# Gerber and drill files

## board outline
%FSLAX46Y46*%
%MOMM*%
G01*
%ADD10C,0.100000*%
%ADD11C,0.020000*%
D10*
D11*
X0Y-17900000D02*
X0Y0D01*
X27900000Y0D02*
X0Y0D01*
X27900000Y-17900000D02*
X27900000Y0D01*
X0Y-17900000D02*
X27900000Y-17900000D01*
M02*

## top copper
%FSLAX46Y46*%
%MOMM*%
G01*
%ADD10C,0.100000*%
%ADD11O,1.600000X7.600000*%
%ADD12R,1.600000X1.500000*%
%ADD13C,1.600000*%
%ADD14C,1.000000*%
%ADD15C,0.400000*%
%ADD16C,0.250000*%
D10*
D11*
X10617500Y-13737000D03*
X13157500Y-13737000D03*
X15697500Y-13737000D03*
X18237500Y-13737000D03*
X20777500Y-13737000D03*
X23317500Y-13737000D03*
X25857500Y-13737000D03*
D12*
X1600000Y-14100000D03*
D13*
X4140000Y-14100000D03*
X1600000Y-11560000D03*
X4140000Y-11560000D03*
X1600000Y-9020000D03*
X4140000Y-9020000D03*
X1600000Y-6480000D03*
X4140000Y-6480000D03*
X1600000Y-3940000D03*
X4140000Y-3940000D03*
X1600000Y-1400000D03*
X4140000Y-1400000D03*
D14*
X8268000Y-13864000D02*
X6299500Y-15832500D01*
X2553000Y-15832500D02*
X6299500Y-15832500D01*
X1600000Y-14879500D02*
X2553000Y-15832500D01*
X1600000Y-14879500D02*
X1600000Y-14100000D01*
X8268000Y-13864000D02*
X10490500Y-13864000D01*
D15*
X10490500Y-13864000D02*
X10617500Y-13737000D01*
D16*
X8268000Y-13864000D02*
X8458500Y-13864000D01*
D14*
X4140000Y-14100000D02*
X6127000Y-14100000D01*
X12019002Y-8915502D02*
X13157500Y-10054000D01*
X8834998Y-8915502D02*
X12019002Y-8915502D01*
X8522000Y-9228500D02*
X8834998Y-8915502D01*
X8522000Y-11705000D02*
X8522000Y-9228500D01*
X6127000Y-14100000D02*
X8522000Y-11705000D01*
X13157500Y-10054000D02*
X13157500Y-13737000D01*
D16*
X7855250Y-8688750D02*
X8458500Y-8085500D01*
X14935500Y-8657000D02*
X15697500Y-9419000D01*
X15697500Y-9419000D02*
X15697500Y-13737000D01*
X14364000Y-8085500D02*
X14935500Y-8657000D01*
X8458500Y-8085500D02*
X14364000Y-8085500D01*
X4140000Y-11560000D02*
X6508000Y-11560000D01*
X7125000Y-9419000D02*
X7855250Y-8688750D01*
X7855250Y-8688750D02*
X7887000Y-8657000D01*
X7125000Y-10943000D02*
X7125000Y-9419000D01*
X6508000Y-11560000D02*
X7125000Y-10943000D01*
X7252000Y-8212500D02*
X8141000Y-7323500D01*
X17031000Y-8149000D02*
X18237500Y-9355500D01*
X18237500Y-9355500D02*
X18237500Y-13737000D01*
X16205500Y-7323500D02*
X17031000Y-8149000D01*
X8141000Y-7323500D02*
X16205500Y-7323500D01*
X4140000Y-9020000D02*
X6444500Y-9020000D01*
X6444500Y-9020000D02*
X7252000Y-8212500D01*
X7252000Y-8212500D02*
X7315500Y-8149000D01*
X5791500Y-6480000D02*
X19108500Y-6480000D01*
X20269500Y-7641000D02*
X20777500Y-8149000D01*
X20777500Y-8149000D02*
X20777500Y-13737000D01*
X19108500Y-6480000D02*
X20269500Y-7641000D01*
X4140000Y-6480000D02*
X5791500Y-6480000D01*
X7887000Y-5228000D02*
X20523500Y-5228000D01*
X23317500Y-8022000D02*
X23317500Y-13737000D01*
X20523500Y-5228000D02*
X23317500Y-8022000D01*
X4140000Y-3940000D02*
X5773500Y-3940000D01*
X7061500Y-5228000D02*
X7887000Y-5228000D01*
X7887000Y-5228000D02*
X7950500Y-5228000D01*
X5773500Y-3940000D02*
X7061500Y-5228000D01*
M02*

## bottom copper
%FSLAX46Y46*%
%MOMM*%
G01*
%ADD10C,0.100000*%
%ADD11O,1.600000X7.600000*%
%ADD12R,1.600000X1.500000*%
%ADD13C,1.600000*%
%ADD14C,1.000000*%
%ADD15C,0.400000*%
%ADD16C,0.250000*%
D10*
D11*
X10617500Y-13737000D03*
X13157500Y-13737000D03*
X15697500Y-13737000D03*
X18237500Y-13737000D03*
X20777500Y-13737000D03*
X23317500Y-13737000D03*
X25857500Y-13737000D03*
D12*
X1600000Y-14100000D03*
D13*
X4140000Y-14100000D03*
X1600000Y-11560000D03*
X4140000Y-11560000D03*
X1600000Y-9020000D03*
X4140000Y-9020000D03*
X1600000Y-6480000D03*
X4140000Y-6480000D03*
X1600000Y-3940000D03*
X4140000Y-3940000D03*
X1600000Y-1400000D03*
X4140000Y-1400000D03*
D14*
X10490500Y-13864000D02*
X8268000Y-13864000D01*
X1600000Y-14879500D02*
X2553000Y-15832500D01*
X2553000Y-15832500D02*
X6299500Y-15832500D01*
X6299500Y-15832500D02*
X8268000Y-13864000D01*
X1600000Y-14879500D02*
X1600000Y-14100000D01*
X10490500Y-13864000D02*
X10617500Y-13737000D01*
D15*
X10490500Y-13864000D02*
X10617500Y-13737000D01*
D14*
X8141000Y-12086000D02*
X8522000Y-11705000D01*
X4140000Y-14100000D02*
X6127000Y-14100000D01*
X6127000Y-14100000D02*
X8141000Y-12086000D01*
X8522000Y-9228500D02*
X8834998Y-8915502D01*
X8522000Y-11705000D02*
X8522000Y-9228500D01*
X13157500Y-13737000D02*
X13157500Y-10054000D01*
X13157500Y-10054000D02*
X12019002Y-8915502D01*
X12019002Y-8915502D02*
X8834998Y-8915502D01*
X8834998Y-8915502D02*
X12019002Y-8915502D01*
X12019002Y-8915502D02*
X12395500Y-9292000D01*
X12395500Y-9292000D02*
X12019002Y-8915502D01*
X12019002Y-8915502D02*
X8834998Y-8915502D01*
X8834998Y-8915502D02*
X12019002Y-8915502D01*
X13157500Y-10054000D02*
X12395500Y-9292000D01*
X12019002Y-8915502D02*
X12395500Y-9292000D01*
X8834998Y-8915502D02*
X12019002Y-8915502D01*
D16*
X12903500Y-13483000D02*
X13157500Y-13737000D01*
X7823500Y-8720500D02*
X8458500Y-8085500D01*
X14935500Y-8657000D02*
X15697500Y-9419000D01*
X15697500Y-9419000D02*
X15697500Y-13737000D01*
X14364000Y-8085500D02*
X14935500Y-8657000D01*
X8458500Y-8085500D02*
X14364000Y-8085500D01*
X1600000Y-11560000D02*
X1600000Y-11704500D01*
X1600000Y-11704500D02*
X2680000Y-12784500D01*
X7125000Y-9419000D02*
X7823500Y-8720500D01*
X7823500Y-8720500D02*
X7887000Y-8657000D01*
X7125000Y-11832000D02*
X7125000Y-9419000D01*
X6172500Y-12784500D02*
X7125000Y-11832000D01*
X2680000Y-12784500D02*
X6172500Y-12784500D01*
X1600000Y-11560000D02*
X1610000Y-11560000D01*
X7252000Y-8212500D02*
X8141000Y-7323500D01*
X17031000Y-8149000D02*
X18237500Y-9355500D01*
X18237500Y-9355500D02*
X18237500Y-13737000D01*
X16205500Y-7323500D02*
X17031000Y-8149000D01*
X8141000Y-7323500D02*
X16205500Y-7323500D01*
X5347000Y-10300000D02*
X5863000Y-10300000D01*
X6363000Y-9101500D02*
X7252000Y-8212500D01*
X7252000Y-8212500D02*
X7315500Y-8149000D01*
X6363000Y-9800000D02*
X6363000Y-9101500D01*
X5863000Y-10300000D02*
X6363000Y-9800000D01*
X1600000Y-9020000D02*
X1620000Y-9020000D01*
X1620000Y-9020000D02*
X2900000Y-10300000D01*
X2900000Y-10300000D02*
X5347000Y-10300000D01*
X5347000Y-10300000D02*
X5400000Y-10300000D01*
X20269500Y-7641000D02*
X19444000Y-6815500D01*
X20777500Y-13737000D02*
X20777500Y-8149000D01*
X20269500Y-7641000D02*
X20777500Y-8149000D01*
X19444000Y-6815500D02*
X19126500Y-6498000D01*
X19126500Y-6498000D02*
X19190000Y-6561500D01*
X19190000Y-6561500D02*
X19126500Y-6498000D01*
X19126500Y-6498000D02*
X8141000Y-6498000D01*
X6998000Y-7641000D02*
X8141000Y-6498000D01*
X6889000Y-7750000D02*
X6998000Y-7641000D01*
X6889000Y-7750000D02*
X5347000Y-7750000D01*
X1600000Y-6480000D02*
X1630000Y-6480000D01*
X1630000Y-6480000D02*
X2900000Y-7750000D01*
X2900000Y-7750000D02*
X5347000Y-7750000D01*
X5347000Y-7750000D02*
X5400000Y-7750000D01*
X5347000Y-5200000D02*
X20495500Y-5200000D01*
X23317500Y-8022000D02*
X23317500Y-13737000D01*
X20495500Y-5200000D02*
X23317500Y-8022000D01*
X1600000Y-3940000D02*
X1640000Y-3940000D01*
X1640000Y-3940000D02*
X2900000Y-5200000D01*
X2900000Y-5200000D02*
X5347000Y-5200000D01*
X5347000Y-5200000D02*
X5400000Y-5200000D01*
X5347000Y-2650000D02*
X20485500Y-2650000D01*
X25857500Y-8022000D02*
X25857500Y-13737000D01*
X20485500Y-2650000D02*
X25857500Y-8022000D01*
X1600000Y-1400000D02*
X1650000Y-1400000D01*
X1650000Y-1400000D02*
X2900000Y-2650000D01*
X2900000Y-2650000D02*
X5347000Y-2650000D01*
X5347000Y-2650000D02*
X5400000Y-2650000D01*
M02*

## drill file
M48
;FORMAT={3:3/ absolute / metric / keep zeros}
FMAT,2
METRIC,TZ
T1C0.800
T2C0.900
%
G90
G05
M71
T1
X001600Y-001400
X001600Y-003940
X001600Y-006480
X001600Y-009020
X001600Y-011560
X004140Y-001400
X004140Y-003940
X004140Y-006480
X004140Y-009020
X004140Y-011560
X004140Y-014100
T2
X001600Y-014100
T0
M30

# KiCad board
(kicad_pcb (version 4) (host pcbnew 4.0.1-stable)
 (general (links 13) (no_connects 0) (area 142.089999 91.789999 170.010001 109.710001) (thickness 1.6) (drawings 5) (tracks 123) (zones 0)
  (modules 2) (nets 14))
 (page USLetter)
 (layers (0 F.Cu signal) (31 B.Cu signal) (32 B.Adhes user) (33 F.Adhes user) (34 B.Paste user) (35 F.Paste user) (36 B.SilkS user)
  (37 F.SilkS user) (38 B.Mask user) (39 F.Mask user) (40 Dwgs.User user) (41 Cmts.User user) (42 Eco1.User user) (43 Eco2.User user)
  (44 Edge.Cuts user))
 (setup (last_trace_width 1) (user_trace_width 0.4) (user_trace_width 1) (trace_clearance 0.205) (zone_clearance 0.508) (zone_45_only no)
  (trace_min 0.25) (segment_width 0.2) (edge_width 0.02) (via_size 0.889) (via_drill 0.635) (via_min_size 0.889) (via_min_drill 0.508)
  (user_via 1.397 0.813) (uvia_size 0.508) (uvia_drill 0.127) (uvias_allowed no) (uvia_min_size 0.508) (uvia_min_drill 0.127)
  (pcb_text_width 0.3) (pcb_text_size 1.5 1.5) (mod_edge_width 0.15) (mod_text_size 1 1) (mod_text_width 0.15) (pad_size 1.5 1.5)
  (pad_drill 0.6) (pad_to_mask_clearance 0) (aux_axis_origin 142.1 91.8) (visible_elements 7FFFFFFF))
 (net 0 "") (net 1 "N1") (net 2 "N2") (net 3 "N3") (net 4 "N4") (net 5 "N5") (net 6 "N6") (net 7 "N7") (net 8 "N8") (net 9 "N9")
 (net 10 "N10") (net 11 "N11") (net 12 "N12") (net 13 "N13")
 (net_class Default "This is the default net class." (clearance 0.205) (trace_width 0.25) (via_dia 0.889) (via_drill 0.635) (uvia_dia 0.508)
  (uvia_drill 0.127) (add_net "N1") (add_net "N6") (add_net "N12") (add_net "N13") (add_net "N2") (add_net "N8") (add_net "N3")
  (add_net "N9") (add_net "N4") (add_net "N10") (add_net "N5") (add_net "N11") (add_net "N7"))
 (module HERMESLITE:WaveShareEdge (layer F.Cu) (at 152.7175 105.537 90)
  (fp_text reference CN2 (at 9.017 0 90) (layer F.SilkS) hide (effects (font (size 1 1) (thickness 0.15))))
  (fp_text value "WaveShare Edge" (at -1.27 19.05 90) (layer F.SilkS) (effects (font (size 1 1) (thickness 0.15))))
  (pad 1 smd oval (at 0 0 90) (size 7.6 1.6) (layers F.Cu F.Paste F.Mask) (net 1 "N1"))
  (pad 3 smd oval (at 0 2.54 90) (size 7.6 1.6) (layers F.Cu F.Paste F.Mask) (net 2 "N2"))
  (pad 5 smd oval (at 0 5.08 90) (size 7.6 1.6) (layers F.Cu F.Paste F.Mask) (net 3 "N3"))
  (pad 7 smd oval (at 0 7.62 90) (size 7.6 1.6) (layers F.Cu F.Paste F.Mask) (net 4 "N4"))
  (pad 9 smd oval (at 0 10.16 90) (size 7.6 1.6) (layers F.Cu F.Paste F.Mask) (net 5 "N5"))
  (pad 11 smd oval (at 0 12.7 90) (size 7.6 1.6) (layers F.Cu F.Paste F.Mask) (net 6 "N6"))
  (pad 13 smd oval (at 0 15.24 90) (size 7.6 1.6) (layers F.Cu F.Paste F.Mask) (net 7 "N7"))
  (pad 2 smd oval (at 0 0 90) (size 7.6 1.6) (layers B.Cu B.Paste B.Mask) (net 1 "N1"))
  (pad 4 smd oval (at 0 2.54 90) (size 7.6 1.6) (layers B.Cu B.Paste B.Mask) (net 2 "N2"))
  (pad 6 smd oval (at 0 5.08 90) (size 7.6 1.6) (layers B.Cu B.Paste B.Mask) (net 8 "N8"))
  (pad 8 smd oval (at 0 7.62 90) (size 7.6 1.6) (layers B.Cu B.Paste B.Mask) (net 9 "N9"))
  (pad 10 smd oval (at 0 10.16 90) (size 7.6 1.6) (layers B.Cu B.Paste B.Mask) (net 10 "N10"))
  (pad 12 smd oval (at 0 12.7 90) (size 7.6 1.6) (layers B.Cu B.Paste B.Mask) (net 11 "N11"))
  (pad 14 smd oval (at 0 15.24 90) (size 7.6 1.6) (layers B.Cu B.Paste B.Mask) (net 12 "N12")))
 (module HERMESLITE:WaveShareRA (layer F.Cu) (at 143.7 105.9)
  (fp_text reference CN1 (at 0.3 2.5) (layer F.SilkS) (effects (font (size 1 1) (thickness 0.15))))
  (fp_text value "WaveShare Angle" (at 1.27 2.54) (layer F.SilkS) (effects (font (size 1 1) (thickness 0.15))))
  (pad 1 thru_hole rect (at 0 0) (size 1.6 1.5) (drill 0.9) (layers *.Cu *.Mask F.SilkS) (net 1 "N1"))
  (pad 2 thru_hole circle (at 2.54 0) (size 1.6 1.6) (drill 0.8) (layers *.Cu *.Mask F.SilkS) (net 2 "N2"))
  (pad 3 thru_hole circle (at 0 -2.54) (size 1.6 1.6) (drill 0.8) (layers *.Cu *.Mask F.SilkS) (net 8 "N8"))
  (pad 4 thru_hole circle (at 2.54 -2.54) (size 1.6 1.6) (drill 0.8) (layers *.Cu *.Mask F.SilkS) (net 3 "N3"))
  (pad 5 thru_hole circle (at 0 -5.08) (size 1.6 1.6) (drill 0.8) (layers *.Cu *.Mask F.SilkS) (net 9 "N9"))
  (pad 6 thru_hole circle (at 2.54 -5.08) (size 1.6 1.6) (drill 0.8) (layers *.Cu *.Mask F.SilkS) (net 4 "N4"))
  (pad 7 thru_hole circle (at 0 -7.62) (size 1.6 1.6) (drill 0.8) (layers *.Cu *.Mask F.SilkS) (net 10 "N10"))
  (pad 8 thru_hole circle (at 2.54 -7.62) (size 1.6 1.6) (drill 0.8) (layers *.Cu *.Mask F.SilkS) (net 5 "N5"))
  (pad 9 thru_hole circle (at 0 -10.16) (size 1.6 1.6) (drill 0.8) (layers *.Cu *.Mask F.SilkS) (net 11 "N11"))
  (pad 10 thru_hole circle (at 2.54 -10.16) (size 1.6 1.6) (drill 0.8) (layers *.Cu *.Mask F.SilkS) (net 6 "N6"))
  (pad 11 thru_hole circle (at 0 -12.7) (size 1.6 1.6) (drill 0.8) (layers *.Cu *.Mask F.SilkS) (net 12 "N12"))
  (pad 12 thru_hole circle (at 2.54 -12.7) (size 1.6 1.6) (drill 0.8) (layers *.Cu *.Mask F.SilkS) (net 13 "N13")))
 (gr_line (start 142.1 109.7) (end 142.1 91.8) (angle 90) (layer Edge.Cuts) (width 0.02))
 (gr_line (start 170 91.8) (end 142.1 91.8) (angle 90) (layer Edge.Cuts) (width 0.02))
 (gr_line (start 170 109.7) (end 170 91.8) (angle 90) (layer Edge.Cuts) (width 0.02))
 (gr_line (start 142.1 109.7) (end 170 109.7) (angle 90) (layer Edge.Cuts) (width 0.02))
 (segment (start 152.5905 105.664) (end 150.368 105.664) (width 1) (layer B.Cu) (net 1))
 (segment (start 143.7 106.6795) (end 144.653 107.6325) (width 1) (layer B.Cu) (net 1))
 (segment (start 144.653 107.6325) (end 148.3995 107.6325) (width 1) (layer B.Cu) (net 1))
 (segment (start 148.3995 107.6325) (end 150.368 105.664) (width 1) (layer B.Cu) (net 1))
 (segment (start 143.7 106.6795) (end 143.7 105.9) (width 1) (layer B.Cu) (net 1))
 (segment (start 152.5905 105.664) (end 152.7175 105.537) (width 1) (layer B.Cu) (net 1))
 (segment (start 152.5905 105.664) (end 152.7175 105.537) (width 0.4) (layer B.Cu) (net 1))
 (segment (start 150.368 105.664) (end 148.3995 107.6325) (width 1) (layer F.Cu) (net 1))
 (segment (start 144.653 107.6325) (end 148.3995 107.6325) (width 1) (layer F.Cu) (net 1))
 (segment (start 143.7 106.6795) (end 144.653 107.6325) (width 1) (layer F.Cu) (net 1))
 (segment (start 143.7 106.6795) (end 143.7 105.9) (width 1) (layer F.Cu) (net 1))
 (segment (start 150.368 105.664) (end 152.5905 105.664) (width 1) (layer F.Cu) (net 1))
 (segment (start 152.5905 105.664) (end 152.7175 105.537) (width 0.4) (layer F.Cu) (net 1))
 (segment (start 150.368 105.664) (end 150.5585 105.664) (width 0.25) (layer F.Cu) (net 1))
 (segment (start 146.24 105.9) (end 148.227 105.9) (width 1) (layer F.Cu) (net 2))
 (segment (start 154.119002 100.715502) (end 155.2575 101.854) (width 1) (layer F.Cu) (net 2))
 (segment (start 150.934998 100.715502) (end 154.119002 100.715502) (width 1) (layer F.Cu) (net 2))
 (segment (start 150.622 101.0285) (end 150.934998 100.715502) (width 1) (layer F.Cu) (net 2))
 (segment (start 150.622 103.505) (end 150.622 101.0285) (width 1) (layer F.Cu) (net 2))
 (segment (start 148.227 105.9) (end 150.622 103.505) (width 1) (layer F.Cu) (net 2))
 (segment (start 155.2575 101.854) (end 155.2575 105.537) (width 1) (layer F.Cu) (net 2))
 (segment (start 150.241 103.886) (end 150.622 103.505) (width 1) (layer B.Cu) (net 2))
 (segment (start 146.24 105.9) (end 148.227 105.9) (width 1) (layer B.Cu) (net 2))
 (segment (start 148.227 105.9) (end 150.241 103.886) (width 1) (layer B.Cu) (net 2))
 (segment (start 150.622 101.0285) (end 150.934998 100.715502) (width 1) (layer B.Cu) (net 2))
 (segment (start 150.622 103.505) (end 150.622 101.0285) (width 1) (layer B.Cu) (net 2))
 (segment (start 155.2575 105.537) (end 155.2575 101.854) (width 1) (layer B.Cu) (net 2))
 (segment (start 155.2575 101.854) (end 154.119002 100.715502) (width 1) (layer B.Cu) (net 2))
 (segment (start 154.119002 100.715502) (end 150.934998 100.715502) (width 1) (layer B.Cu) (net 2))
 (segment (start 150.934998 100.715502) (end 154.119002 100.715502) (width 1) (layer B.Cu) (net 2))
 (segment (start 154.119002 100.715502) (end 154.4955 101.092) (width 1) (layer B.Cu) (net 2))
 (segment (start 154.4955 101.092) (end 154.119002 100.715502) (width 1) (layer B.Cu) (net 2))
 (segment (start 154.119002 100.715502) (end 150.934998 100.715502) (width 1) (layer B.Cu) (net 2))
 (segment (start 150.934998 100.715502) (end 154.119002 100.715502) (width 1) (layer B.Cu) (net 2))
 (segment (start 155.2575 101.854) (end 154.4955 101.092) (width 1) (layer B.Cu) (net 2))
 (segment (start 154.119002 100.715502) (end 154.4955 101.092) (width 1) (layer B.Cu) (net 2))
 (segment (start 150.934998 100.715502) (end 154.119002 100.715502) (width 1) (layer B.Cu) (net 2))
 (segment (start 155.0035 105.283) (end 155.2575 105.537) (width 0.25) (layer B.Cu) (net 2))
 (segment (start 149.9235 100.5205) (end 150.5585 99.8855) (width 0.25) (layer B.Cu) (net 8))
 (segment (start 157.0355 100.457) (end 157.7975 101.219) (width 0.25) (layer B.Cu) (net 8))
 (segment (start 157.7975 101.219) (end 157.7975 105.537) (width 0.25) (layer B.Cu) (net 8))
 (segment (start 156.464 99.8855) (end 157.0355 100.457) (width 0.25) (layer B.Cu) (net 8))
 (segment (start 150.5585 99.8855) (end 156.464 99.8855) (width 0.25) (layer B.Cu) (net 8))
 (segment (start 143.7 103.36) (end 143.7 103.5045) (width 0.25) (layer B.Cu) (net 8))
 (segment (start 143.7 103.5045) (end 144.78 104.5845) (width 0.25) (layer B.Cu) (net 8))
 (segment (start 149.225 101.219) (end 149.9235 100.5205) (width 0.25) (layer B.Cu) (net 8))
 (segment (start 149.9235 100.5205) (end 149.987 100.457) (width 0.25) (layer B.Cu) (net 8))
 (segment (start 149.225 103.632) (end 149.225 101.219) (width 0.25) (layer B.Cu) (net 8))
 (segment (start 148.2725 104.5845) (end 149.225 103.632) (width 0.25) (layer B.Cu) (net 8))
 (segment (start 144.78 104.5845) (end 148.2725 104.5845) (width 0.25) (layer B.Cu) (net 8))
 (segment (start 143.7 103.36) (end 143.71 103.36) (width 0.25) (layer B.Cu) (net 8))
 (segment (start 149.95525 100.48875) (end 150.5585 99.8855) (width 0.25) (layer F.Cu) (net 3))
 (segment (start 157.0355 100.457) (end 157.7975 101.219) (width 0.25) (layer F.Cu) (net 3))
 (segment (start 157.7975 101.219) (end 157.7975 105.537) (width 0.25) (layer F.Cu) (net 3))
 (segment (start 156.464 99.8855) (end 157.0355 100.457) (width 0.25) (layer F.Cu) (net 3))
 (segment (start 150.5585 99.8855) (end 156.464 99.8855) (width 0.25) (layer F.Cu) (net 3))
 (segment (start 146.24 103.36) (end 148.608 103.36) (width 0.25) (layer F.Cu) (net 3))
 (segment (start 149.225 101.219) (end 149.95525 100.48875) (width 0.25) (layer F.Cu) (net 3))
 (segment (start 149.95525 100.48875) (end 149.987 100.457) (width 0.25) (layer F.Cu) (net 3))
 (segment (start 149.225 102.743) (end 149.225 101.219) (width 0.25) (layer F.Cu) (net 3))
 (segment (start 148.608 103.36) (end 149.225 102.743) (width 0.25) (layer F.Cu) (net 3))
 (segment (start 149.352 100.0125) (end 150.241 99.1235) (width 0.25) (layer B.Cu) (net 9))
 (segment (start 159.131 99.949) (end 160.3375 101.1555) (width 0.25) (layer B.Cu) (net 9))
 (segment (start 160.3375 101.1555) (end 160.3375 105.537) (width 0.25) (layer B.Cu) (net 9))
 (segment (start 158.3055 99.1235) (end 159.131 99.949) (width 0.25) (layer B.Cu) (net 9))
 (segment (start 150.241 99.1235) (end 158.3055 99.1235) (width 0.25) (layer B.Cu) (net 9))
 (segment (start 147.447 102.1) (end 147.963 102.1) (width 0.25) (layer B.Cu) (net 9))
 (segment (start 148.463 100.9015) (end 149.352 100.0125) (width 0.25) (layer B.Cu) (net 9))
 (segment (start 149.352 100.0125) (end 149.4155 99.949) (width 0.25) (layer B.Cu) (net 9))
 (segment (start 148.463 101.6) (end 148.463 100.9015) (width 0.25) (layer B.Cu) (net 9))
 (segment (start 147.963 102.1) (end 148.463 101.6) (width 0.25) (layer B.Cu) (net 9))
 (segment (start 143.7 100.82) (end 143.72 100.82) (width 0.25) (layer B.Cu) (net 9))
 (segment (start 143.72 100.82) (end 145 102.1) (width 0.25) (layer B.Cu) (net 9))
 (segment (start 145 102.1) (end 147.447 102.1) (width 0.25) (layer B.Cu) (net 9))
 (segment (start 147.447 102.1) (end 147.5 102.1) (width 0.25) (layer B.Cu) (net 9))
 (segment (start 149.352 100.0125) (end 150.241 99.1235) (width 0.25) (layer F.Cu) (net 4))
 (segment (start 159.131 99.949) (end 160.3375 101.1555) (width 0.25) (layer F.Cu) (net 4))
 (segment (start 160.3375 101.1555) (end 160.3375 105.537) (width 0.25) (layer F.Cu) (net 4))
 (segment (start 158.3055 99.1235) (end 159.131 99.949) (width 0.25) (layer F.Cu) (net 4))
 (segment (start 150.241 99.1235) (end 158.3055 99.1235) (width 0.25) (layer F.Cu) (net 4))
 (segment (start 146.24 100.82) (end 148.5445 100.82) (width 0.25) (layer F.Cu) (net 4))
 (segment (start 148.5445 100.82) (end 149.352 100.0125) (width 0.25) (layer F.Cu) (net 4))
 (segment (start 149.352 100.0125) (end 149.4155 99.949) (width 0.25) (layer F.Cu) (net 4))
 (segment (start 162.3695 99.441) (end 161.544 98.6155) (width 0.25) (layer B.Cu) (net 10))
 (segment (start 162.8775 105.537) (end 162.8775 99.949) (width 0.25) (layer B.Cu) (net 10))
 (segment (start 162.3695 99.441) (end 162.8775 99.949) (width 0.25) (layer B.Cu) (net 10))
 (segment (start 161.544 98.6155) (end 161.2265 98.298) (width 0.25) (layer B.Cu) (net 10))
 (segment (start 161.2265 98.298) (end 161.29 98.3615) (width 0.25) (layer B.Cu) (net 10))
 (segment (start 161.29 98.3615) (end 161.2265 98.298) (width 0.25) (layer B.Cu) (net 10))
 (segment (start 161.2265 98.298) (end 150.241 98.298) (width 0.25) (layer B.Cu) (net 10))
 (segment (start 149.098 99.441) (end 150.241 98.298) (width 0.25) (layer B.Cu) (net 10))
 (segment (start 148.989 99.55) (end 149.098 99.441) (width 0.25) (layer B.Cu) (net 10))
 (segment (start 148.989 99.55) (end 147.447 99.55) (width 0.25) (layer B.Cu) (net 10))
 (segment (start 143.7 98.28) (end 143.73 98.28) (width 0.25) (layer B.Cu) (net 10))
 (segment (start 143.73 98.28) (end 145 99.55) (width 0.25) (layer B.Cu) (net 10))
 (segment (start 145 99.55) (end 147.447 99.55) (width 0.25) (layer B.Cu) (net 10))
 (segment (start 147.447 99.55) (end 147.5 99.55) (width 0.25) (layer B.Cu) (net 10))
 (segment (start 147.8915 98.28) (end 161.2085 98.28) (width 0.25) (layer F.Cu) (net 5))
 (segment (start 162.3695 99.441) (end 162.8775 99.949) (width 0.25) (layer F.Cu) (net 5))
 (segment (start 162.8775 99.949) (end 162.8775 105.537) (width 0.25) (layer F.Cu) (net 5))
 (segment (start 161.2085 98.28) (end 162.3695 99.441) (width 0.25) (layer F.Cu) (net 5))
 (segment (start 146.24 98.28) (end 147.8915 98.28) (width 0.25) (layer F.Cu) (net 5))
 (segment (start 147.447 97) (end 162.5955 97) (width 0.25) (layer B.Cu) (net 11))
 (segment (start 165.4175 99.822) (end 165.4175 105.537) (width 0.25) (layer B.Cu) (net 11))
 (segment (start 162.5955 97) (end 165.4175 99.822) (width 0.25) (layer B.Cu) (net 11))
 (segment (start 143.7 95.74) (end 143.74 95.74) (width 0.25) (layer B.Cu) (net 11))
 (segment (start 143.74 95.74) (end 145 97) (width 0.25) (layer B.Cu) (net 11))
 (segment (start 145 97) (end 147.447 97) (width 0.25) (layer B.Cu) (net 11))
 (segment (start 147.447 97) (end 147.5 97) (width 0.25) (layer B.Cu) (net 11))
 (segment (start 149.987 97.028) (end 162.6235 97.028) (width 0.25) (layer F.Cu) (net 6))
 (segment (start 165.4175 99.822) (end 165.4175 105.537) (width 0.25) (layer F.Cu) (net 6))
 (segment (start 162.6235 97.028) (end 165.4175 99.822) (width 0.25) (layer F.Cu) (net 6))
 (segment (start 146.24 95.74) (end 147.8735 95.74) (width 0.25) (layer F.Cu) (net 6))
 (segment (start 149.1615 97.028) (end 149.987 97.028) (width 0.25) (layer F.Cu) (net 6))
 (segment (start 149.987 97.028) (end 150.0505 97.028) (width 0.25) (layer F.Cu) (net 6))
 (segment (start 147.8735 95.74) (end 149.1615 97.028) (width 0.25) (layer F.Cu) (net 6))
 (segment (start 147.447 94.45) (end 162.5855 94.45) (width 0.25) (layer B.Cu) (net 12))
 (segment (start 167.9575 99.822) (end 167.9575 105.537) (width 0.25) (layer B.Cu) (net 12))
 (segment (start 162.5855 94.45) (end 167.9575 99.822) (width 0.25) (layer B.Cu) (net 12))
 (segment (start 143.7 93.2) (end 143.75 93.2) (width 0.25) (layer B.Cu) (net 12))
 (segment (start 143.75 93.2) (end 145 94.45) (width 0.25) (layer B.Cu) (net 12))
 (segment (start 145 94.45) (end 147.447 94.45) (width 0.25) (layer B.Cu) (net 12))
 (segment (start 147.447 94.45) (end 147.5 94.45) (width 0.25) (layer B.Cu) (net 12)))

